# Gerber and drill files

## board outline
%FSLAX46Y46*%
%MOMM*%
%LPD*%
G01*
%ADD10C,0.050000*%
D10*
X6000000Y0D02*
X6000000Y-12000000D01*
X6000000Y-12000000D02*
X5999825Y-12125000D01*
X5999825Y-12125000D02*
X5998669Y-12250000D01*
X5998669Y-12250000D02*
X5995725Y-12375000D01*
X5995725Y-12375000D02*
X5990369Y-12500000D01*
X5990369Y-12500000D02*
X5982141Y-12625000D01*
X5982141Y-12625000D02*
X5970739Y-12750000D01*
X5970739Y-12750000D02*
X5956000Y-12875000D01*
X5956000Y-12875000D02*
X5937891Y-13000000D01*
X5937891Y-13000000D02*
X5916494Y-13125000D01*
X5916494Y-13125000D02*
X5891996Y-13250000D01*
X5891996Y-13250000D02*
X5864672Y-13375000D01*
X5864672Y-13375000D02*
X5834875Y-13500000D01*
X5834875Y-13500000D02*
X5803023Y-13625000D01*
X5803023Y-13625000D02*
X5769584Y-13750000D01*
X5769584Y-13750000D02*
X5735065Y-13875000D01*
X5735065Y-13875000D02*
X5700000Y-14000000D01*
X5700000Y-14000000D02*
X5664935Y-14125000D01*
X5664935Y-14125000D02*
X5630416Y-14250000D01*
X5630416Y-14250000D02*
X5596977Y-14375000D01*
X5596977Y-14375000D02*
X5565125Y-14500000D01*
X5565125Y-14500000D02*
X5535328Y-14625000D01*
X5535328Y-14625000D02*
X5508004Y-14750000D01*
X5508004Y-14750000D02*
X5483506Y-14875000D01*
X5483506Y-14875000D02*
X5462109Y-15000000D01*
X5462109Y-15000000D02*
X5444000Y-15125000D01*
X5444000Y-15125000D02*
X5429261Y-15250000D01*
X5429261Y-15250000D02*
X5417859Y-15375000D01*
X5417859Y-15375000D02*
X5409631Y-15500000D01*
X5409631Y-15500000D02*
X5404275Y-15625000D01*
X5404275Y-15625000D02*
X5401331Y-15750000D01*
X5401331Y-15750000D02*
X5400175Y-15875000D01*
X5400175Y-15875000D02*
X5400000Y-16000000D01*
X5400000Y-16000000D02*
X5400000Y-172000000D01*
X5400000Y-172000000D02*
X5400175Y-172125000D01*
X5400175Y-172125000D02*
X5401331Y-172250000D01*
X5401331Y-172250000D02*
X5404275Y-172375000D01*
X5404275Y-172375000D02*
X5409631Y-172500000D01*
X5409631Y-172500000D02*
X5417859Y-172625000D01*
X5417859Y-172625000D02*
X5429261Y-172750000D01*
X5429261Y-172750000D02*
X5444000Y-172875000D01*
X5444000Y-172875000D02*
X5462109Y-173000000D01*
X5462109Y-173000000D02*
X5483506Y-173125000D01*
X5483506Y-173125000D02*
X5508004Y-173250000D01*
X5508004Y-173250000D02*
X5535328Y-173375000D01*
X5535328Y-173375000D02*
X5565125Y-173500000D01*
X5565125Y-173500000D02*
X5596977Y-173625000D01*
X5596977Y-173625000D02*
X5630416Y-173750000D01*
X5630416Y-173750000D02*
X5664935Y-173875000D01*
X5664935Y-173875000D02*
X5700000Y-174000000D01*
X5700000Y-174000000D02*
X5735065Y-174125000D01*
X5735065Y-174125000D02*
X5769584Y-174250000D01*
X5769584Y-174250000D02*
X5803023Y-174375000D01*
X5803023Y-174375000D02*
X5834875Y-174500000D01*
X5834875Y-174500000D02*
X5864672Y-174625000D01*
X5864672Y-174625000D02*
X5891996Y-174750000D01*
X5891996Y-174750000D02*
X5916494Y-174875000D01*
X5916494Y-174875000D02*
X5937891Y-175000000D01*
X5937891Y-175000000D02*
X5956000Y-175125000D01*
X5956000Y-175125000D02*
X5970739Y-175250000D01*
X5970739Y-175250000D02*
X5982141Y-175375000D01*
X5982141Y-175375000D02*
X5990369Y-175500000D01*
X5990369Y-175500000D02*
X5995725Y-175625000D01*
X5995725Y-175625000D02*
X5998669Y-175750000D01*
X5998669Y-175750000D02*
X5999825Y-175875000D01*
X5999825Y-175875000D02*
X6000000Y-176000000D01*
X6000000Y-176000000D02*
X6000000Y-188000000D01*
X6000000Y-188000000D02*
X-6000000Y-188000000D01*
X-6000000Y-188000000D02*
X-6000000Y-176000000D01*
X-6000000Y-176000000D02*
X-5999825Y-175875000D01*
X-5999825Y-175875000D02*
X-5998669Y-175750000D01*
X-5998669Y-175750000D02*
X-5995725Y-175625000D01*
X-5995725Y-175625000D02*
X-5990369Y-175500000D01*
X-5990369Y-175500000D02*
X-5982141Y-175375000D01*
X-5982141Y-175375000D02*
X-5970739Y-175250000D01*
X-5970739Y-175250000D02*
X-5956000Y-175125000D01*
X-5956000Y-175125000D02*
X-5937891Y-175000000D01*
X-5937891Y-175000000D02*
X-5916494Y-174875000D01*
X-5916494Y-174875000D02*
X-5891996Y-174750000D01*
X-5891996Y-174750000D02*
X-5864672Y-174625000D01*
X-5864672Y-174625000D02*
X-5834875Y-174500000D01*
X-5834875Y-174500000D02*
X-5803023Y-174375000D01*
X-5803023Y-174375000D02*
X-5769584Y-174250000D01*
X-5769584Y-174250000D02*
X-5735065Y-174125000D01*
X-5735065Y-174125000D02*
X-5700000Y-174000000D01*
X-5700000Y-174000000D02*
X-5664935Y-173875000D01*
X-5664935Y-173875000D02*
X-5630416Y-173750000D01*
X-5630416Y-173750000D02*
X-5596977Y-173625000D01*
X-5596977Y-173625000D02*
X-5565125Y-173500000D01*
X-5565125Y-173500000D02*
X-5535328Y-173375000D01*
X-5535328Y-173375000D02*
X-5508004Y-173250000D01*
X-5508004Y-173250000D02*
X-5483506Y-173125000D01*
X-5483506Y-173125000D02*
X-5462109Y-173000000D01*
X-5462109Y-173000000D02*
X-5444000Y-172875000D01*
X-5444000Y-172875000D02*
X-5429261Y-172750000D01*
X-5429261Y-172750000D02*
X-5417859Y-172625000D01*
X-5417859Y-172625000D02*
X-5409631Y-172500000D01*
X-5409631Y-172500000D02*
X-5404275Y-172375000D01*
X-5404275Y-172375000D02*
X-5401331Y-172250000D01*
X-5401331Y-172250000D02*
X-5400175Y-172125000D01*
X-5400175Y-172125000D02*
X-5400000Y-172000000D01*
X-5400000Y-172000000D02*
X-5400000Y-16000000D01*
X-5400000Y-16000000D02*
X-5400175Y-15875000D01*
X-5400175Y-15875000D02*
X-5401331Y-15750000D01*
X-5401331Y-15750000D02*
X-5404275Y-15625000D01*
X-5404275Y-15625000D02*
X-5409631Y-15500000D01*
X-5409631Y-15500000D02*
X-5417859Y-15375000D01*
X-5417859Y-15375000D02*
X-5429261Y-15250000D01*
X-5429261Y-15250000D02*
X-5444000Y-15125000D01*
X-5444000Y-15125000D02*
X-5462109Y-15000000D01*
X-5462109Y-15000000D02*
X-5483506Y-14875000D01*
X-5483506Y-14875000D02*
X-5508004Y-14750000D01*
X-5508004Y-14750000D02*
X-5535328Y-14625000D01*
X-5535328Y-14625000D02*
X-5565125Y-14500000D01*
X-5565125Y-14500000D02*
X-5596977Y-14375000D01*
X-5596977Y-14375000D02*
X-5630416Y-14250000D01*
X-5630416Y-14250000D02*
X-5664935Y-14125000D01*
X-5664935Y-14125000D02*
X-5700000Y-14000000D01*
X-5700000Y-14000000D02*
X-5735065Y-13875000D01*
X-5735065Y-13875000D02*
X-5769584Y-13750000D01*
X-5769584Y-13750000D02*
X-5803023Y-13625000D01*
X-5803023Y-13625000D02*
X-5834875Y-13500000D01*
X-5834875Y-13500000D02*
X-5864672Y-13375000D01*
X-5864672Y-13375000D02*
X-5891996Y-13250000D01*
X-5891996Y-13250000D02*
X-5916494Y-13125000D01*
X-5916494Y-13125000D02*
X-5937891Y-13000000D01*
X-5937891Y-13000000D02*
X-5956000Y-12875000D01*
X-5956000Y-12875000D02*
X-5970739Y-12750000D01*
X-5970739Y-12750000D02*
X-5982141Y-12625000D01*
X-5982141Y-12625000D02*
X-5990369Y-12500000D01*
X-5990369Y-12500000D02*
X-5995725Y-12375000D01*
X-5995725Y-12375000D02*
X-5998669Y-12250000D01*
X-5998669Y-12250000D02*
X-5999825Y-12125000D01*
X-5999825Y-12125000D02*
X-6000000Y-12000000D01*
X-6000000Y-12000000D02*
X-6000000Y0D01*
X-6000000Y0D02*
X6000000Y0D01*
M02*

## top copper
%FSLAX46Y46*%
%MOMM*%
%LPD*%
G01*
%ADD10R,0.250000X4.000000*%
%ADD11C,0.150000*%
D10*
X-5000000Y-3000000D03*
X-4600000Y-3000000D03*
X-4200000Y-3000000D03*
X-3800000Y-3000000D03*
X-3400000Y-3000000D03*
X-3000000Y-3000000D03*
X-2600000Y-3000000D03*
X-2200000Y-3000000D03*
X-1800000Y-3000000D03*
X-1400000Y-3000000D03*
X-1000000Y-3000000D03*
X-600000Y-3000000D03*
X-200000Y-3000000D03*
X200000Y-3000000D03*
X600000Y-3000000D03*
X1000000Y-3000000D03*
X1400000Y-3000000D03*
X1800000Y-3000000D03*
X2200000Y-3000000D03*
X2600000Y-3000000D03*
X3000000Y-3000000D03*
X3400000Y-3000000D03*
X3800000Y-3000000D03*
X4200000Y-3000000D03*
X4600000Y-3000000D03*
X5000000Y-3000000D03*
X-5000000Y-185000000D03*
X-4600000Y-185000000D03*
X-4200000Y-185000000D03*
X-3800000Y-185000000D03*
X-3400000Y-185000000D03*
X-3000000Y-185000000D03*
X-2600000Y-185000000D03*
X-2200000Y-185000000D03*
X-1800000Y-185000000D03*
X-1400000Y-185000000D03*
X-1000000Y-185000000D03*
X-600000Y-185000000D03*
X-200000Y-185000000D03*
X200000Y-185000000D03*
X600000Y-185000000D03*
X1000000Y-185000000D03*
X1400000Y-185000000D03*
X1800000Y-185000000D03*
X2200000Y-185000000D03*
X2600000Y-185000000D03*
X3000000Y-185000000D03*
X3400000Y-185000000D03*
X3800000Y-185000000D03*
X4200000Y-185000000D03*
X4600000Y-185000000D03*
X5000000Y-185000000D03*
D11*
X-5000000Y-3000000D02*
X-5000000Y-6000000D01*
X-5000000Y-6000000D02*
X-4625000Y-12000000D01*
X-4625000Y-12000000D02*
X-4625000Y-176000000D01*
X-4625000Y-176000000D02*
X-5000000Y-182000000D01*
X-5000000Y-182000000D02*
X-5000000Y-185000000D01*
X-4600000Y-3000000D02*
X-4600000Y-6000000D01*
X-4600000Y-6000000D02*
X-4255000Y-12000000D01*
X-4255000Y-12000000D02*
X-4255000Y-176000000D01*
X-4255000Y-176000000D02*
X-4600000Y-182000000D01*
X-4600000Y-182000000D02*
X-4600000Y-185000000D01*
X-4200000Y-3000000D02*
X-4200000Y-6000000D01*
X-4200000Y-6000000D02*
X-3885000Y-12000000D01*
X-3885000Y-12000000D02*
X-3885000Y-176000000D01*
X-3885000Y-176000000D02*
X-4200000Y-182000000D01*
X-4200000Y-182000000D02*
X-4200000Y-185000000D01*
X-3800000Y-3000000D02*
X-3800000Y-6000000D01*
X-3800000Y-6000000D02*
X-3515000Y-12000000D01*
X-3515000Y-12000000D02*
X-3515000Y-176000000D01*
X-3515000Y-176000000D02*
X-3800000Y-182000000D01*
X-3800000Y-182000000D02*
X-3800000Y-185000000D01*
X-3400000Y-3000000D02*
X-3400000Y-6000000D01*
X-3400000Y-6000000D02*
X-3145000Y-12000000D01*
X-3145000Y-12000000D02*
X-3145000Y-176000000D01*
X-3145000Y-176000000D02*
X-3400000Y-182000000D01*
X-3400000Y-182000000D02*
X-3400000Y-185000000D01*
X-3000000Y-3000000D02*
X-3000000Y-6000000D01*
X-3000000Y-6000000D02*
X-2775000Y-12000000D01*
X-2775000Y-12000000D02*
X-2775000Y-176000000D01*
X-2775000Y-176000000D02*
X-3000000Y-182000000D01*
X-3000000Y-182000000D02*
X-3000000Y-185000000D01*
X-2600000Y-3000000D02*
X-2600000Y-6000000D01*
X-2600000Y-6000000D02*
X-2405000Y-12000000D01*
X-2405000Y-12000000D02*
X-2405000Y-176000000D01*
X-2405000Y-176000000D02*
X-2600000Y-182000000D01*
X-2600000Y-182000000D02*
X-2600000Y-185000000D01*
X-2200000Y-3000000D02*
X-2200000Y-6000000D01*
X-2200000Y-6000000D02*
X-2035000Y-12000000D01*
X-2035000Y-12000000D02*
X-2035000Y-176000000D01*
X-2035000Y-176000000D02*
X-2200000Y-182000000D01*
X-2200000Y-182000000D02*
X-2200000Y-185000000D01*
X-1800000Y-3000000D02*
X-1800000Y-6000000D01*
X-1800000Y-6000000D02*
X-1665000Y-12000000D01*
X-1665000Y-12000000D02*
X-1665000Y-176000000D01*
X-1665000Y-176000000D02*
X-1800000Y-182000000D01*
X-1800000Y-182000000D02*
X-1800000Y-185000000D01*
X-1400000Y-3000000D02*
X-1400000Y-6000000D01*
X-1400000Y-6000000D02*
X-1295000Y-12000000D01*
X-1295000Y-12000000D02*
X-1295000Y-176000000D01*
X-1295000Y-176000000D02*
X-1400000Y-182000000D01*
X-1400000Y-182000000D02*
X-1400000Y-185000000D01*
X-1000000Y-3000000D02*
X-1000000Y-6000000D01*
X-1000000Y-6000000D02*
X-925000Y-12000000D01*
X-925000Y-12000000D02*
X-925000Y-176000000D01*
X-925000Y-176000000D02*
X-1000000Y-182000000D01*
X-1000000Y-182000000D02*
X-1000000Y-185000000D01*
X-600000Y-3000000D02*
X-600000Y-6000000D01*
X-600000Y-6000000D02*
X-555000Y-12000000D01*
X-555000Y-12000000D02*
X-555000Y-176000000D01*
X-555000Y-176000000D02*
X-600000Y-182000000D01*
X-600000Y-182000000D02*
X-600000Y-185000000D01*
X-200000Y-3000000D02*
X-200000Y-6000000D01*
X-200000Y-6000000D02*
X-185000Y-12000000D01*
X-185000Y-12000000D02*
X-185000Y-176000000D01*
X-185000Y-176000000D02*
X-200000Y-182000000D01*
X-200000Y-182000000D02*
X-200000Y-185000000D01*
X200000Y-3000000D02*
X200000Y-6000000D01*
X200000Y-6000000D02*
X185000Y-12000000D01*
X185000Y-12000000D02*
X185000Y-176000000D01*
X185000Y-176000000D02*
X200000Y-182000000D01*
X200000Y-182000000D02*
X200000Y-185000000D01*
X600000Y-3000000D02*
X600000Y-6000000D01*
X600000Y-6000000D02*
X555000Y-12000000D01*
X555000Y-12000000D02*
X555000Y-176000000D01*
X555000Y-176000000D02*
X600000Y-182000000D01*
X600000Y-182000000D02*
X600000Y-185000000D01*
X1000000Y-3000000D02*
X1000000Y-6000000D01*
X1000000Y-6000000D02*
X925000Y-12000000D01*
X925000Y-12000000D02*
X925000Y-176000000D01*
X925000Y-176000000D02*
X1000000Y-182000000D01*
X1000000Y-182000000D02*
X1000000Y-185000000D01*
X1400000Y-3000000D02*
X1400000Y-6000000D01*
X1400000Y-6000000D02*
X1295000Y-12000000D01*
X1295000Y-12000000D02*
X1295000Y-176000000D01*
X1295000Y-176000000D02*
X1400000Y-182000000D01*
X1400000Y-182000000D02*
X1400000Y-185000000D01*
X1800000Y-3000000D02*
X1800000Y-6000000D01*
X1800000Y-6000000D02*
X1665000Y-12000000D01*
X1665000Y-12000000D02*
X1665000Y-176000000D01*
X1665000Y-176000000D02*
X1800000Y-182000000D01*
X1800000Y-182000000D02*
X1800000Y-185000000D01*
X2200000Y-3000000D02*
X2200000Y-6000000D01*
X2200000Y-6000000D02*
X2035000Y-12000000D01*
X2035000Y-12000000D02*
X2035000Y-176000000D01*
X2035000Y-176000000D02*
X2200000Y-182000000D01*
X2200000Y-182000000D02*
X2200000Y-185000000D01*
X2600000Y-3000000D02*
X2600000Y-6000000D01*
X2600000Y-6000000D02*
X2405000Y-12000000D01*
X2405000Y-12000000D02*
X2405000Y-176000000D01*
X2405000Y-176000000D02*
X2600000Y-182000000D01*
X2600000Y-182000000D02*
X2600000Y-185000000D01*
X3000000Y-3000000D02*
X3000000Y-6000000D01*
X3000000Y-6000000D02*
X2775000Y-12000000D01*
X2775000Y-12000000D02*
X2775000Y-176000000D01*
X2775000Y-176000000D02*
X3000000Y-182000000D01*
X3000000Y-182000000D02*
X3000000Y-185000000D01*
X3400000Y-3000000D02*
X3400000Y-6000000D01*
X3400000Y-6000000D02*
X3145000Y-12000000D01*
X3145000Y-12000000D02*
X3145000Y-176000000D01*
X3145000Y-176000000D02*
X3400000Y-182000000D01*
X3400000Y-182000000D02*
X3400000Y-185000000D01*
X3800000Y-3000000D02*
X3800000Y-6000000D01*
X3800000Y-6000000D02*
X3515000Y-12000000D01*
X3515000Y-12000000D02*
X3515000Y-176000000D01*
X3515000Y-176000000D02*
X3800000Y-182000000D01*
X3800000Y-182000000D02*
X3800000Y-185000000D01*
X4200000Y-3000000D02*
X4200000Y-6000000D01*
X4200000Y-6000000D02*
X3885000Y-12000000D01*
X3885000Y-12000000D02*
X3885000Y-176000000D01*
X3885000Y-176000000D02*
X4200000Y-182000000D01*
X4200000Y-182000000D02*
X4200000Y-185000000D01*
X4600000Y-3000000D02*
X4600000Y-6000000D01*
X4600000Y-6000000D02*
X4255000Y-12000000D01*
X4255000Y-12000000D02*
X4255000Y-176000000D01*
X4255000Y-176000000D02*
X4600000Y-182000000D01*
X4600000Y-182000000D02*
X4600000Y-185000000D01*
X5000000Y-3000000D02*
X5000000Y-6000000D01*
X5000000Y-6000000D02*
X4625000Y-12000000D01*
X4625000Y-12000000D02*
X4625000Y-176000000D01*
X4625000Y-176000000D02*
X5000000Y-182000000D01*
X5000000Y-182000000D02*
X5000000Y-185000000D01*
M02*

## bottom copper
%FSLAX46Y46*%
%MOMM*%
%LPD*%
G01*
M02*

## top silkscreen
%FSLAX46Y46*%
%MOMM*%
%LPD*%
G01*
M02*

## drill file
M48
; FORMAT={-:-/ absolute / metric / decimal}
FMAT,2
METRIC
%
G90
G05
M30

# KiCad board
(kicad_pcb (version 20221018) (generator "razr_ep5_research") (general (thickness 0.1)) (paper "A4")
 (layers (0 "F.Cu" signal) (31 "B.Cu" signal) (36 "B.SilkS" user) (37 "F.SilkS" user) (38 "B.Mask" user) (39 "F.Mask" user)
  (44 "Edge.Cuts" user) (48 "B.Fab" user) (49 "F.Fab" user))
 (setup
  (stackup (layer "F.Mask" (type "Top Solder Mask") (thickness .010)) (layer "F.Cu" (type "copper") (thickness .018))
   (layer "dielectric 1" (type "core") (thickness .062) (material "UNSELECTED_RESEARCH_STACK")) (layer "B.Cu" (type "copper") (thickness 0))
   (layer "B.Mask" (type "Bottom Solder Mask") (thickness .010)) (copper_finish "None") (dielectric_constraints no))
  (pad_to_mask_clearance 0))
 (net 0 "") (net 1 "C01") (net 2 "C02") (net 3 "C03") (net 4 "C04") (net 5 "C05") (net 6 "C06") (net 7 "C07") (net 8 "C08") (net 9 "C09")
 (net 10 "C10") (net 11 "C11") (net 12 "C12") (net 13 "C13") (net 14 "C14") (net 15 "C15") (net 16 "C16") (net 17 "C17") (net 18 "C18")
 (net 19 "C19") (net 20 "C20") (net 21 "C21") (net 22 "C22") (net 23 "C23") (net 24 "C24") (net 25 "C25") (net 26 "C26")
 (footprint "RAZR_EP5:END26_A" (layer "F.Cu") (at 0 0)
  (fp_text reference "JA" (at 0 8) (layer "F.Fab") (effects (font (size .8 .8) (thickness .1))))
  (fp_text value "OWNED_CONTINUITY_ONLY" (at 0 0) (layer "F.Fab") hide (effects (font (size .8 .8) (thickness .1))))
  (pad "1" smd rect (at -5.0 3.0) (size .25 4) (layers "F.Cu" "F.Mask") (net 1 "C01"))
  (pad "2" smd rect (at -4.6 3.0) (size .25 4) (layers "F.Cu" "F.Mask") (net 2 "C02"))
  (pad "3" smd rect (at -4.2 3.0) (size .25 4) (layers "F.Cu" "F.Mask") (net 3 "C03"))
  (pad "4" smd rect (at -3.8 3.0) (size .25 4) (layers "F.Cu" "F.Mask") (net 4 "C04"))
  (pad "5" smd rect (at -3.4 3.0) (size .25 4) (layers "F.Cu" "F.Mask") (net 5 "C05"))
  (pad "6" smd rect (at -3.0 3.0) (size .25 4) (layers "F.Cu" "F.Mask") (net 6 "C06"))
  (pad "7" smd rect (at -2.6 3.0) (size .25 4) (layers "F.Cu" "F.Mask") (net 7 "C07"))
  (pad "8" smd rect (at -2.2 3.0) (size .25 4) (layers "F.Cu" "F.Mask") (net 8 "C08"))
  (pad "9" smd rect (at -1.8 3.0) (size .25 4) (layers "F.Cu" "F.Mask") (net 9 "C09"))
  (pad "10" smd rect (at -1.4 3.0) (size .25 4) (layers "F.Cu" "F.Mask") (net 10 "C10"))
  (pad "11" smd rect (at -1.0 3.0) (size .25 4) (layers "F.Cu" "F.Mask") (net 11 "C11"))
  (pad "12" smd rect (at -0.6 3.0) (size .25 4) (layers "F.Cu" "F.Mask") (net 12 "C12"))
  (pad "13" smd rect (at -0.2 3.0) (size .25 4) (layers "F.Cu" "F.Mask") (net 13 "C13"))
  (pad "14" smd rect (at 0.2 3.0) (size .25 4) (layers "F.Cu" "F.Mask") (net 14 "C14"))
  (pad "15" smd rect (at 0.6 3.0) (size .25 4) (layers "F.Cu" "F.Mask") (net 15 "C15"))
  (pad "16" smd rect (at 1.0 3.0) (size .25 4) (layers "F.Cu" "F.Mask") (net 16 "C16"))
  (pad "17" smd rect (at 1.4 3.0) (size .25 4) (layers "F.Cu" "F.Mask") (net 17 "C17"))
  (pad "18" smd rect (at 1.8 3.0) (size .25 4) (layers "F.Cu" "F.Mask") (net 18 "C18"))
  (pad "19" smd rect (at 2.2 3.0) (size .25 4) (layers "F.Cu" "F.Mask") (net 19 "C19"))
  (pad "20" smd rect (at 2.6 3.0) (size .25 4) (layers "F.Cu" "F.Mask") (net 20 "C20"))
  (pad "21" smd rect (at 3.0 3.0) (size .25 4) (layers "F.Cu" "F.Mask") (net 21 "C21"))
  (pad "22" smd rect (at 3.4 3.0) (size .25 4) (layers "F.Cu" "F.Mask") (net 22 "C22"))
  (pad "23" smd rect (at 3.8 3.0) (size .25 4) (layers "F.Cu" "F.Mask") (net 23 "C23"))
  (pad "24" smd rect (at 4.2 3.0) (size .25 4) (layers "F.Cu" "F.Mask") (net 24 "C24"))
  (pad "25" smd rect (at 4.6 3.0) (size .25 4) (layers "F.Cu" "F.Mask") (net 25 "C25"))
  (pad "26" smd rect (at 5.0 3.0) (size .25 4) (layers "F.Cu" "F.Mask") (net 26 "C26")))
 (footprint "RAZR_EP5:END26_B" (layer "F.Cu") (at 0 0)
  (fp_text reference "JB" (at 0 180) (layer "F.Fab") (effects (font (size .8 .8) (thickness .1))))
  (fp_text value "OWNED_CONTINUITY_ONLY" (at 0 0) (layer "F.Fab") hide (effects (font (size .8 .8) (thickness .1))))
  (pad "1" smd rect (at -5.0 185.0) (size .25 4) (layers "F.Cu" "F.Mask") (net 1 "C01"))
  (pad "2" smd rect (at -4.6 185.0) (size .25 4) (layers "F.Cu" "F.Mask") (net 2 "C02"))
  (pad "3" smd rect (at -4.2 185.0) (size .25 4) (layers "F.Cu" "F.Mask") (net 3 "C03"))
  (pad "4" smd rect (at -3.8 185.0) (size .25 4) (layers "F.Cu" "F.Mask") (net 4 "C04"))
  (pad "5" smd rect (at -3.4 185.0) (size .25 4) (layers "F.Cu" "F.Mask") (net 5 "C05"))
  (pad "6" smd rect (at -3.0 185.0) (size .25 4) (layers "F.Cu" "F.Mask") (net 6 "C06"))
  (pad "7" smd rect (at -2.6 185.0) (size .25 4) (layers "F.Cu" "F.Mask") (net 7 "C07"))
  (pad "8" smd rect (at -2.2 185.0) (size .25 4) (layers "F.Cu" "F.Mask") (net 8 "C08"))
  (pad "9" smd rect (at -1.8 185.0) (size .25 4) (layers "F.Cu" "F.Mask") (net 9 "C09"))
  (pad "10" smd rect (at -1.4 185.0) (size .25 4) (layers "F.Cu" "F.Mask") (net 10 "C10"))
  (pad "11" smd rect (at -1.0 185.0) (size .25 4) (layers "F.Cu" "F.Mask") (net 11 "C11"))
  (pad "12" smd rect (at -0.6 185.0) (size .25 4) (layers "F.Cu" "F.Mask") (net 12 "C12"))
  (pad "13" smd rect (at -0.2 185.0) (size .25 4) (layers "F.Cu" "F.Mask") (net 13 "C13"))
  (pad "14" smd rect (at 0.2 185.0) (size .25 4) (layers "F.Cu" "F.Mask") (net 14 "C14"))
  (pad "15" smd rect (at 0.6 185.0) (size .25 4) (layers "F.Cu" "F.Mask") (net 15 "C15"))
  (pad "16" smd rect (at 1.0 185.0) (size .25 4) (layers "F.Cu" "F.Mask") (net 16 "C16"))
  (pad "17" smd rect (at 1.4 185.0) (size .25 4) (layers "F.Cu" "F.Mask") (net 17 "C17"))
  (pad "18" smd rect (at 1.8 185.0) (size .25 4) (layers "F.Cu" "F.Mask") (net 18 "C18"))
  (pad "19" smd rect (at 2.2 185.0) (size .25 4) (layers "F.Cu" "F.Mask") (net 19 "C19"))
  (pad "20" smd rect (at 2.6 185.0) (size .25 4) (layers "F.Cu" "F.Mask") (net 20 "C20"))
  (pad "21" smd rect (at 3.0 185.0) (size .25 4) (layers "F.Cu" "F.Mask") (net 21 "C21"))
  (pad "22" smd rect (at 3.4 185.0) (size .25 4) (layers "F.Cu" "F.Mask") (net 22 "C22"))
  (pad "23" smd rect (at 3.8 185.0) (size .25 4) (layers "F.Cu" "F.Mask") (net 23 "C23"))
  (pad "24" smd rect (at 4.2 185.0) (size .25 4) (layers "F.Cu" "F.Mask") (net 24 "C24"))
  (pad "25" smd rect (at 4.6 185.0) (size .25 4) (layers "F.Cu" "F.Mask") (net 25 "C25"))
  (pad "26" smd rect (at 5.0 185.0) (size .25 4) (layers "F.Cu" "F.Mask") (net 26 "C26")))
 (segment (start -5.0 3.0) (end -5.0 6.0) (width .15) (layer "F.Cu") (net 1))
 (segment (start -5.0 6.0) (end -4.625 12) (width .15) (layer "F.Cu") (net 1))
 (segment (start -4.625 12) (end -4.625 176) (width .15) (layer "F.Cu") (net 1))
 (segment (start -4.625 176) (end -5.0 182.0) (width .15) (layer "F.Cu") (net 1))
 (segment (start -5.0 182.0) (end -5.0 185.0) (width .15) (layer "F.Cu") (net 1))
 (segment (start -4.6 3.0) (end -4.6 6.0) (width .15) (layer "F.Cu") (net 2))
 (segment (start -4.6 6.0) (end -4.255 12) (width .15) (layer "F.Cu") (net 2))
 (segment (start -4.255 12) (end -4.255 176) (width .15) (layer "F.Cu") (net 2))
 (segment (start -4.255 176) (end -4.6 182.0) (width .15) (layer "F.Cu") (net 2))
 (segment (start -4.6 182.0) (end -4.6 185.0) (width .15) (layer "F.Cu") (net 2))
 (segment (start -4.2 3.0) (end -4.2 6.0) (width .15) (layer "F.Cu") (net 3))
 (segment (start -4.2 6.0) (end -3.885 12) (width .15) (layer "F.Cu") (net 3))
 (segment (start -3.885 12) (end -3.885 176) (width .15) (layer "F.Cu") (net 3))
 (segment (start -3.885 176) (end -4.2 182.0) (width .15) (layer "F.Cu") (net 3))
 (segment (start -4.2 182.0) (end -4.2 185.0) (width .15) (layer "F.Cu") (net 3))
 (segment (start -3.8 3.0) (end -3.8 6.0) (width .15) (layer "F.Cu") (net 4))
 (segment (start -3.8 6.0) (end -3.515 12) (width .15) (layer "F.Cu") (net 4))
 (segment (start -3.515 12) (end -3.515 176) (width .15) (layer "F.Cu") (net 4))
 (segment (start -3.515 176) (end -3.8 182.0) (width .15) (layer "F.Cu") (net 4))
 (segment (start -3.8 182.0) (end -3.8 185.0) (width .15) (layer "F.Cu") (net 4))
 (segment (start -3.4 3.0) (end -3.4 6.0) (width .15) (layer "F.Cu") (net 5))
 (segment (start -3.4 6.0) (end -3.145 12) (width .15) (layer "F.Cu") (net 5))
 (segment (start -3.145 12) (end -3.145 176) (width .15) (layer "F.Cu") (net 5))
 (segment (start -3.145 176) (end -3.4 182.0) (width .15) (layer "F.Cu") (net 5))
 (segment (start -3.4 182.0) (end -3.4 185.0) (width .15) (layer "F.Cu") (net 5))
 (segment (start -3.0 3.0) (end -3.0 6.0) (width .15) (layer "F.Cu") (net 6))
 (segment (start -3.0 6.0) (end -2.775 12) (width .15) (layer "F.Cu") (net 6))
 (segment (start -2.775 12) (end -2.775 176) (width .15) (layer "F.Cu") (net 6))
 (segment (start -2.775 176) (end -3.0 182.0) (width .15) (layer "F.Cu") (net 6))
 (segment (start -3.0 182.0) (end -3.0 185.0) (width .15) (layer "F.Cu") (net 6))
 (segment (start -2.6 3.0) (end -2.6 6.0) (width .15) (layer "F.Cu") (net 7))
 (segment (start -2.6 6.0) (end -2.405 12) (width .15) (layer "F.Cu") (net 7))
 (segment (start -2.405 12) (end -2.405 176) (width .15) (layer "F.Cu") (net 7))
 (segment (start -2.405 176) (end -2.6 182.0) (width .15) (layer "F.Cu") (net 7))
 (segment (start -2.6 182.0) (end -2.6 185.0) (width .15) (layer "F.Cu") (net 7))
 (segment (start -2.2 3.0) (end -2.2 6.0) (width .15) (layer "F.Cu") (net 8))
 (segment (start -2.2 6.0) (end -2.035 12) (width .15) (layer "F.Cu") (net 8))
 (segment (start -2.035 12) (end -2.035 176) (width .15) (layer "F.Cu") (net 8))
 (segment (start -2.035 176) (end -2.2 182.0) (width .15) (layer "F.Cu") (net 8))
 (segment (start -2.2 182.0) (end -2.2 185.0) (width .15) (layer "F.Cu") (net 8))
 (segment (start -1.8 3.0) (end -1.8 6.0) (width .15) (layer "F.Cu") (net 9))
 (segment (start -1.8 6.0) (end -1.665 12) (width .15) (layer "F.Cu") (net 9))
 (segment (start -1.665 12) (end -1.665 176) (width .15) (layer "F.Cu") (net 9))
 (segment (start -1.665 176) (end -1.8 182.0) (width .15) (layer "F.Cu") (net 9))
 (segment (start -1.8 182.0) (end -1.8 185.0) (width .15) (layer "F.Cu") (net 9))
 (segment (start -1.4 3.0) (end -1.4 6.0) (width .15) (layer "F.Cu") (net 10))
 (segment (start -1.4 6.0) (end -1.295 12) (width .15) (layer "F.Cu") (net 10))
 (segment (start -1.295 12) (end -1.295 176) (width .15) (layer "F.Cu") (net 10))
 (segment (start -1.295 176) (end -1.4 182.0) (width .15) (layer "F.Cu") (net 10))
 (segment (start -1.4 182.0) (end -1.4 185.0) (width .15) (layer "F.Cu") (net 10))
 (segment (start -1.0 3.0) (end -1.0 6.0) (width .15) (layer "F.Cu") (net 11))
 (segment (start -1.0 6.0) (end -0.925 12) (width .15) (layer "F.Cu") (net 11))
 (segment (start -0.925 12) (end -0.925 176) (width .15) (layer "F.Cu") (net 11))
 (segment (start -0.925 176) (end -1.0 182.0) (width .15) (layer "F.Cu") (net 11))
 (segment (start -1.0 182.0) (end -1.0 185.0) (width .15) (layer "F.Cu") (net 11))
 (segment (start -0.6 3.0) (end -0.6 6.0) (width .15) (layer "F.Cu") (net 12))
 (segment (start -0.6 6.0) (end -0.555 12) (width .15) (layer "F.Cu") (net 12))
 (segment (start -0.555 12) (end -0.555 176) (width .15) (layer "F.Cu") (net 12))
 (segment (start -0.555 176) (end -0.6 182.0) (width .15) (layer "F.Cu") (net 12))
 (segment (start -0.6 182.0) (end -0.6 185.0) (width .15) (layer "F.Cu") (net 12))
 (segment (start -0.2 3.0) (end -0.2 6.0) (width .15) (layer "F.Cu") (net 13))
 (segment (start -0.2 6.0) (end -0.185 12) (width .15) (layer "F.Cu") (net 13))
 (segment (start -0.185 12) (end -0.185 176) (width .15) (layer "F.Cu") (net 13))
 (segment (start -0.185 176) (end -0.2 182.0) (width .15) (layer "F.Cu") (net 13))
 (segment (start -0.2 182.0) (end -0.2 185.0) (width .15) (layer "F.Cu") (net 13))
 (segment (start 0.2 3.0) (end 0.2 6.0) (width .15) (layer "F.Cu") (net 14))
 (segment (start 0.2 6.0) (end 0.185 12) (width .15) (layer "F.Cu") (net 14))
 (segment (start 0.185 12) (end 0.185 176) (width .15) (layer "F.Cu") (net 14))
 (segment (start 0.185 176) (end 0.2 182.0) (width .15) (layer "F.Cu") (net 14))
 (segment (start 0.2 182.0) (end 0.2 185.0) (width .15) (layer "F.Cu") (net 14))
 (segment (start 0.6 3.0) (end 0.6 6.0) (width .15) (layer "F.Cu") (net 15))
 (segment (start 0.6 6.0) (end 0.555 12) (width .15) (layer "F.Cu") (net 15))
 (segment (start 0.555 12) (end 0.555 176) (width .15) (layer "F.Cu") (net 15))
 (segment (start 0.555 176) (end 0.6 182.0) (width .15) (layer "F.Cu") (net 15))
 (segment (start 0.6 182.0) (end 0.6 185.0) (width .15) (layer "F.Cu") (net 15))
 (segment (start 1.0 3.0) (end 1.0 6.0) (width .15) (layer "F.Cu") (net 16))
 (segment (start 1.0 6.0) (end 0.925 12) (width .15) (layer "F.Cu") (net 16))
 (segment (start 0.925 12) (end 0.925 176) (width .15) (layer "F.Cu") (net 16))
 (segment (start 0.925 176) (end 1.0 182.0) (width .15) (layer "F.Cu") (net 16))
 (segment (start 1.0 182.0) (end 1.0 185.0) (width .15) (layer "F.Cu") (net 16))
 (segment (start 1.4 3.0) (end 1.4 6.0) (width .15) (layer "F.Cu") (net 17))
 (segment (start 1.4 6.0) (end 1.295 12) (width .15) (layer "F.Cu") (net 17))
 (segment (start 1.295 12) (end 1.295 176) (width .15) (layer "F.Cu") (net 17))
 (segment (start 1.295 176) (end 1.4 182.0) (width .15) (layer "F.Cu") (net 17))
 (segment (start 1.4 182.0) (end 1.4 185.0) (width .15) (layer "F.Cu") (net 17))
 (segment (start 1.8 3.0) (end 1.8 6.0) (width .15) (layer "F.Cu") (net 18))
 (segment (start 1.8 6.0) (end 1.665 12) (width .15) (layer "F.Cu") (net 18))
 (segment (start 1.665 12) (end 1.665 176) (width .15) (layer "F.Cu") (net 18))
 (segment (start 1.665 176) (end 1.8 182.0) (width .15) (layer "F.Cu") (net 18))
 (segment (start 1.8 182.0) (end 1.8 185.0) (width .15) (layer "F.Cu") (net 18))
 (segment (start 2.2 3.0) (end 2.2 6.0) (width .15) (layer "F.Cu") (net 19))
 (segment (start 2.2 6.0) (end 2.035 12) (width .15) (layer "F.Cu") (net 19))
 (segment (start 2.035 12) (end 2.035 176) (width .15) (layer "F.Cu") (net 19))
 (segment (start 2.035 176) (end 2.2 182.0) (width .15) (layer "F.Cu") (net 19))
 (segment (start 2.2 182.0) (end 2.2 185.0) (width .15) (layer "F.Cu") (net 19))
 (segment (start 2.6 3.0) (end 2.6 6.0) (width .15) (layer "F.Cu") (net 20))
 (segment (start 2.6 6.0) (end 2.405 12) (width .15) (layer "F.Cu") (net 20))
 (segment (start 2.405 12) (end 2.405 176) (width .15) (layer "F.Cu") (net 20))
 (segment (start 2.405 176) (end 2.6 182.0) (width .15) (layer "F.Cu") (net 20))
 (segment (start 2.6 182.0) (end 2.6 185.0) (width .15) (layer "F.Cu") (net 20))
 (segment (start 3.0 3.0) (end 3.0 6.0) (width .15) (layer "F.Cu") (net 21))
 (segment (start 3.0 6.0) (end 2.775 12) (width .15) (layer "F.Cu") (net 21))
 (segment (start 2.775 12) (end 2.775 176) (width .15) (layer "F.Cu") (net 21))
 (segment (start 2.775 176) (end 3.0 182.0) (width .15) (layer "F.Cu") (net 21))
 (segment (start 3.0 182.0) (end 3.0 185.0) (width .15) (layer "F.Cu") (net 21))
 (segment (start 3.4 3.0) (end 3.4 6.0) (width .15) (layer "F.Cu") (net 22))
 (segment (start 3.4 6.0) (end 3.145 12) (width .15) (layer "F.Cu") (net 22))
 (segment (start 3.145 12) (end 3.145 176) (width .15) (layer "F.Cu") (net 22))
 (segment (start 3.145 176) (end 3.4 182.0) (width .15) (layer "F.Cu") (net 22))
 (segment (start 3.4 182.0) (end 3.4 185.0) (width .15) (layer "F.Cu") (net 22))
 (segment (start 3.8 3.0) (end 3.8 6.0) (width .15) (layer "F.Cu") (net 23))
 (segment (start 3.8 6.0) (end 3.515 12) (width .15) (layer "F.Cu") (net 23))
 (segment (start 3.515 12) (end 3.515 176) (width .15) (layer "F.Cu") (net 23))
 (segment (start 3.515 176) (end 3.8 182.0) (width .15) (layer "F.Cu") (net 23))
 (segment (start 3.8 182.0) (end 3.8 185.0) (width .15) (layer "F.Cu") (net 23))
 (segment (start 4.2 3.0) (end 4.2 6.0) (width .15) (layer "F.Cu") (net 24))
 (segment (start 4.2 6.0) (end 3.885 12) (width .15) (layer "F.Cu") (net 24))
 (segment (start 3.885 12) (end 3.885 176) (width .15) (layer "F.Cu") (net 24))
 (segment (start 3.885 176) (end 4.2 182.0) (width .15) (layer "F.Cu") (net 24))
 (segment (start 4.2 182.0) (end 4.2 185.0) (width .15) (layer "F.Cu") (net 24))
 (segment (start 4.6 3.0) (end 4.6 6.0) (width .15) (layer "F.Cu") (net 25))
 (segment (start 4.6 6.0) (end 4.255 12) (width .15) (layer "F.Cu") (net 25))
 (segment (start 4.255 12) (end 4.255 176) (width .15) (layer "F.Cu") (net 25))
 (segment (start 4.255 176) (end 4.6 182.0) (width .15) (layer "F.Cu") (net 25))
 (segment (start 4.6 182.0) (end 4.6 185.0) (width .15) (layer "F.Cu") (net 25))
 (segment (start 5.0 3.0) (end 5.0 6.0) (width .15) (layer "F.Cu") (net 26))
 (segment (start 5.0 6.0) (end 4.625 12) (width .15) (layer "F.Cu") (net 26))
 (segment (start 4.625 12) (end 4.625 176) (width .15) (layer "F.Cu") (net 26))
 (segment (start 4.625 176) (end 5.0 182.0) (width .15) (layer "F.Cu") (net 26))
 (segment (start 5.0 182.0) (end 5.0 185.0) (width .15) (layer "F.Cu") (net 26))
 (gr_line (start 6.0 0.0) (end 6.0 12) (layer "Edge.Cuts") (width .05))
 (gr_line (start 6.0 12) (end 5.99982537 12.125) (layer "Edge.Cuts") (width .05))
 (gr_line (start 5.99982537 12.125) (end 5.998669052 12.25) (layer "Edge.Cuts") (width .05))
 (gr_line (start 5.998669052 12.25) (end 5.99572531 12.375) (layer "Edge.Cuts") (width .05))
 (gr_line (start 5.99572531 12.375) (end 5.990368652 12.5) (layer "Edge.Cuts") (width .05))
 (gr_line (start 5.990368652 12.5) (end 5.982140958 12.625) (layer "Edge.Cuts") (width .05))
 (gr_line (start 5.982140958 12.625) (end 5.970738602 12.75) (layer "Edge.Cuts") (width .05))
 (gr_line (start 5.970738602 12.75) (end 5.955999577 12.875) (layer "Edge.Cuts") (width .05))
 (gr_line (start 5.955999577 12.875) (end 5.937890625 13.0) (layer "Edge.Cuts") (width .05))
 (gr_line (start 5.937890625 13.0) (end 5.916494358 13.125) (layer "Edge.Cuts") (width .05))
 (gr_line (start 5.916494358 13.125) (end 5.891996384 13.25) (layer "Edge.Cuts") (width .05))
 (gr_line (start 5.891996384 13.25) (end 5.864672434 13.375) (layer "Edge.Cuts") (width .05))
 (gr_line (start 5.864672434 13.375) (end 5.834875488 13.5) (layer "Edge.Cuts") (width .05))
 (gr_line (start 5.834875488 13.5) (end 5.803022897 13.625) (layer "Edge.Cuts") (width .05))
 (gr_line (start 5.803022897 13.625) (end 5.769583511 13.75) (layer "Edge.Cuts") (width .05))
 (gr_line (start 5.769583511 13.75) (end 5.735064805 13.875) (layer "Edge.Cuts") (width .05))
 (gr_line (start 5.735064805 13.875) (end 5.7 14.0) (layer "Edge.Cuts") (width .05))
 (gr_line (start 5.7 14.0) (end 5.664935195 14.125) (layer "Edge.Cuts") (width .05))
 (gr_line (start 5.664935195 14.125) (end 5.630416489 14.25) (layer "Edge.Cuts") (width .05))
 (gr_line (start 5.630416489 14.25) (end 5.596977103 14.375) (layer "Edge.Cuts") (width .05))
 (gr_line (start 5.596977103 14.375) (end 5.565124512 14.5) (layer "Edge.Cuts") (width .05))
 (gr_line (start 5.565124512 14.5) (end 5.535327566 14.625) (layer "Edge.Cuts") (width .05))
 (gr_line (start 5.535327566 14.625) (end 5.508003616 14.75) (layer "Edge.Cuts") (width .05))
 (gr_line (start 5.508003616 14.75) (end 5.483505642 14.875) (layer "Edge.Cuts") (width .05))
 (gr_line (start 5.483505642 14.875) (end 5.462109375 15.0) (layer "Edge.Cuts") (width .05))
 (gr_line (start 5.462109375 15.0) (end 5.444000423 15.125) (layer "Edge.Cuts") (width .05))
 (gr_line (start 5.444000423 15.125) (end 5.429261398 15.25) (layer "Edge.Cuts") (width .05))
 (gr_line (start 5.429261398 15.25) (end 5.417859042 15.375) (layer "Edge.Cuts") (width .05))
 (gr_line (start 5.417859042 15.375) (end 5.409631348 15.5) (layer "Edge.Cuts") (width .05))
 (gr_line (start 5.409631348 15.5) (end 5.40427469 15.625) (layer "Edge.Cuts") (width .05))
 (gr_line (start 5.40427469 15.625) (end 5.401330948 15.75) (layer "Edge.Cuts") (width .05))
 (gr_line (start 5.401330948 15.75) (end 5.40017463 15.875) (layer "Edge.Cuts") (width .05))
 (gr_line (start 5.40017463 15.875) (end 5.4 16.0) (layer "Edge.Cuts") (width .05))
 (gr_line (start 5.4 16.0) (end 5.4 172.0) (layer "Edge.Cuts") (width .05))
 (gr_line (start 5.4 172.0) (end 5.40017463 172.125) (layer "Edge.Cuts") (width .05))
 (gr_line (start 5.40017463 172.125) (end 5.401330948 172.25) (layer "Edge.Cuts") (width .05))
 (gr_line (start 5.401330948 172.25) (end 5.40427469 172.375) (layer "Edge.Cuts") (width .05))
 (gr_line (start 5.40427469 172.375) (end 5.409631348 172.5) (layer "Edge.Cuts") (width .05))
 (gr_line (start 5.409631348 172.5) (end 5.417859042 172.625) (layer "Edge.Cuts") (width .05))
 (gr_line (start 5.417859042 172.625) (end 5.429261398 172.75) (layer "Edge.Cuts") (width .05))
 (gr_line (start 5.429261398 172.75) (end 5.444000423 172.875) (layer "Edge.Cuts") (width .05))
 (gr_line (start 5.444000423 172.875) (end 5.462109375 173.0) (layer "Edge.Cuts") (width .05))
 (gr_line (start 5.462109375 173.0) (end 5.483505642 173.125) (layer "Edge.Cuts") (width .05))
 (gr_line (start 5.483505642 173.125) (end 5.508003616 173.25) (layer "Edge.Cuts") (width .05))
 (gr_line (start 5.508003616 173.25) (end 5.535327566 173.375) (layer "Edge.Cuts") (width .05))
 (gr_line (start 5.535327566 173.375) (end 5.565124512 173.5) (layer "Edge.Cuts") (width .05))
 (gr_line (start 5.565124512 173.5) (end 5.596977103 173.625) (layer "Edge.Cuts") (width .05))
 (gr_line (start 5.596977103 173.625) (end 5.630416489 173.75) (layer "Edge.Cuts") (width .05))
 (gr_line (start 5.630416489 173.75) (end 5.664935195 173.875) (layer "Edge.Cuts") (width .05))
 (gr_line (start 5.664935195 173.875) (end 5.7 174.0) (layer "Edge.Cuts") (width .05))
 (gr_line (start 5.7 174.0) (end 5.735064805 174.125) (layer "Edge.Cuts") (width .05))
 (gr_line (start 5.735064805 174.125) (end 5.769583511 174.25) (layer "Edge.Cuts") (width .05))
 (gr_line (start 5.769583511 174.25) (end 5.803022897 174.375) (layer "Edge.Cuts") (width .05))
 (gr_line (start 5.803022897 174.375) (end 5.834875488 174.5) (layer "Edge.Cuts") (width .05))
 (gr_line (start 5.834875488 174.5) (end 5.864672434 174.625) (layer "Edge.Cuts") (width .05))
 (gr_line (start 5.864672434 174.625) (end 5.891996384 174.75) (layer "Edge.Cuts") (width .05))
 (gr_line (start 5.891996384 174.75) (end 5.916494358 174.875) (layer "Edge.Cuts") (width .05))
 (gr_line (start 5.916494358 174.875) (end 5.937890625 175.0) (layer "Edge.Cuts") (width .05))
 (gr_line (start 5.937890625 175.0) (end 5.955999577 175.125) (layer "Edge.Cuts") (width .05))
 (gr_line (start 5.955999577 175.125) (end 5.970738602 175.25) (layer "Edge.Cuts") (width .05))
 (gr_line (start 5.970738602 175.25) (end 5.982140958 175.375) (layer "Edge.Cuts") (width .05))
 (gr_line (start 5.982140958 175.375) (end 5.990368652 175.5) (layer "Edge.Cuts") (width .05))
 (gr_line (start 5.990368652 175.5) (end 5.99572531 175.625) (layer "Edge.Cuts") (width .05))
 (gr_line (start 5.99572531 175.625) (end 5.998669052 175.75) (layer "Edge.Cuts") (width .05))
 (gr_line (start 5.998669052 175.75) (end 5.99982537 175.875) (layer "Edge.Cuts") (width .05))
 (gr_line (start 5.99982537 175.875) (end 6.0 176) (layer "Edge.Cuts") (width .05))
 (gr_line (start 6.0 176) (end 6.0 188) (layer "Edge.Cuts") (width .05))
 (gr_line (start 6.0 188) (end -6.0 188) (layer "Edge.Cuts") (width .05))
 (gr_line (start -6.0 188) (end -6.0 176) (layer "Edge.Cuts") (width .05))
 (gr_line (start -6.0 176) (end -5.99982537 175.875) (layer "Edge.Cuts") (width .05))
 (gr_line (start -5.99982537 175.875) (end -5.998669052 175.75) (layer "Edge.Cuts") (width .05))
 (gr_line (start -5.998669052 175.75) (end -5.99572531 175.625) (layer "Edge.Cuts") (width .05))
 (gr_line (start -5.99572531 175.625) (end -5.990368652 175.5) (layer "Edge.Cuts") (width .05))
 (gr_line (start -5.990368652 175.5) (end -5.982140958 175.375) (layer "Edge.Cuts") (width .05))
 (gr_line (start -5.982140958 175.375) (end -5.970738602 175.25) (layer "Edge.Cuts") (width .05))
 (gr_line (start -5.970738602 175.25) (end -5.955999577 175.125) (layer "Edge.Cuts") (width .05))
 (gr_line (start -5.955999577 175.125) (end -5.937890625 175.0) (layer "Edge.Cuts") (width .05))
 (gr_line (start -5.937890625 175.0) (end -5.916494358 174.875) (layer "Edge.Cuts") (width .05))
 (gr_line (start -5.916494358 174.875) (end -5.891996384 174.75) (layer "Edge.Cuts") (width .05))
 (gr_line (start -5.891996384 174.75) (end -5.864672434 174.625) (layer "Edge.Cuts") (width .05))
 (gr_line (start -5.864672434 174.625) (end -5.834875488 174.5) (layer "Edge.Cuts") (width .05))
 (gr_line (start -5.834875488 174.5) (end -5.803022897 174.375) (layer "Edge.Cuts") (width .05))
 (gr_line (start -5.803022897 174.375) (end -5.769583511 174.25) (layer "Edge.Cuts") (width .05))
 (gr_line (start -5.769583511 174.25) (end -5.735064805 174.125) (layer "Edge.Cuts") (width .05))
 (gr_line (start -5.735064805 174.125) (end -5.7 174.0) (layer "Edge.Cuts") (width .05))
 (gr_line (start -5.7 174.0) (end -5.664935195 173.875) (layer "Edge.Cuts") (width .05))
 (gr_line (start -5.664935195 173.875) (end -5.630416489 173.75) (layer "Edge.Cuts") (width .05))
 (gr_line (start -5.630416489 173.75) (end -5.596977103 173.625) (layer "Edge.Cuts") (width .05))
 (gr_line (start -5.596977103 173.625) (end -5.565124512 173.5) (layer "Edge.Cuts") (width .05))
 (gr_line (start -5.565124512 173.5) (end -5.535327566 173.375) (layer "Edge.Cuts") (width .05))
 (gr_line (start -5.535327566 173.375) (end -5.508003616 173.25) (layer "Edge.Cuts") (width .05))
 (gr_line (start -5.508003616 173.25) (end -5.483505642 173.125) (layer "Edge.Cuts") (width .05))
 (gr_line (start -5.483505642 173.125) (end -5.462109375 173.0) (layer "Edge.Cuts") (width .05))
 (gr_line (start -5.462109375 173.0) (end -5.444000423 172.875) (layer "Edge.Cuts") (width .05))
 (gr_line (start -5.444000423 172.875) (end -5.429261398 172.75) (layer "Edge.Cuts") (width .05))
 (gr_line (start -5.429261398 172.75) (end -5.417859042 172.625) (layer "Edge.Cuts") (width .05))
 (gr_line (start -5.417859042 172.625) (end -5.409631348 172.5) (layer "Edge.Cuts") (width .05))
 (gr_line (start -5.409631348 172.5) (end -5.40427469 172.375) (layer "Edge.Cuts") (width .05))
 (gr_line (start -5.40427469 172.375) (end -5.401330948 172.25) (layer "Edge.Cuts") (width .05))
 (gr_line (start -5.401330948 172.25) (end -5.40017463 172.125) (layer "Edge.Cuts") (width .05))
 (gr_line (start -5.40017463 172.125) (end -5.4 172.0) (layer "Edge.Cuts") (width .05))
 (gr_line (start -5.4 172.0) (end -5.4 16.0) (layer "Edge.Cuts") (width .05))
 (gr_line (start -5.4 16.0) (end -5.40017463 15.875) (layer "Edge.Cuts") (width .05))
 (gr_line (start -5.40017463 15.875) (end -5.401330948 15.75) (layer "Edge.Cuts") (width .05))
 (gr_line (start -5.401330948 15.75) (end -5.40427469 15.625) (layer "Edge.Cuts") (width .05))
 (gr_line (start -5.40427469 15.625) (end -5.409631348 15.5) (layer "Edge.Cuts") (width .05))
 (gr_line (start -5.409631348 15.5) (end -5.417859042 15.375) (layer "Edge.Cuts") (width .05))
 (gr_line (start -5.417859042 15.375) (end -5.429261398 15.25) (layer "Edge.Cuts") (width .05))
 (gr_line (start -5.429261398 15.25) (end -5.444000423 15.125) (layer "Edge.Cuts") (width .05))
 (gr_line (start -5.444000423 15.125) (end -5.462109375 15.0) (layer "Edge.Cuts") (width .05))
 (gr_line (start -5.462109375 15.0) (end -5.483505642 14.875) (layer "Edge.Cuts") (width .05))
 (gr_line (start -5.483505642 14.875) (end -5.508003616 14.75) (layer "Edge.Cuts") (width .05))
 (gr_line (start -5.508003616 14.75) (end -5.535327566 14.625) (layer "Edge.Cuts") (width .05))
 (gr_line (start -5.535327566 14.625) (end -5.565124512 14.5) (layer "Edge.Cuts") (width .05))
 (gr_line (start -5.565124512 14.5) (end -5.596977103 14.375) (layer "Edge.Cuts") (width .05))
 (gr_line (start -5.596977103 14.375) (end -5.630416489 14.25) (layer "Edge.Cuts") (width .05))
 (gr_line (start -5.630416489 14.25) (end -5.664935195 14.125) (layer "Edge.Cuts") (width .05))
 (gr_line (start -5.664935195 14.125) (end -5.7 14.0) (layer "Edge.Cuts") (width .05))
 (gr_line (start -5.7 14.0) (end -5.735064805 13.875) (layer "Edge.Cuts") (width .05))
 (gr_line (start -5.735064805 13.875) (end -5.769583511 13.75) (layer "Edge.Cuts") (width .05))
 (gr_line (start -5.769583511 13.75) (end -5.803022897 13.625) (layer "Edge.Cuts") (width .05))
 (gr_line (start -5.803022897 13.625) (end -5.834875488 13.5) (layer "Edge.Cuts") (width .05))
 (gr_line (start -5.834875488 13.5) (end -5.864672434 13.375) (layer "Edge.Cuts") (width .05))
 (gr_line (start -5.864672434 13.375) (end -5.891996384 13.25) (layer "Edge.Cuts") (width .05))
 (gr_line (start -5.891996384 13.25) (end -5.916494358 13.125) (layer "Edge.Cuts") (width .05))
 (gr_line (start -5.916494358 13.125) (end -5.937890625 13.0) (layer "Edge.Cuts") (width .05))
 (gr_line (start -5.937890625 13.0) (end -5.955999577 12.875) (layer "Edge.Cuts") (width .05))
 (gr_line (start -5.955999577 12.875) (end -5.970738602 12.75) (layer "Edge.Cuts") (width .05))
 (gr_line (start -5.970738602 12.75) (end -5.982140958 12.625) (layer "Edge.Cuts") (width .05))
 (gr_line (start -5.982140958 12.625) (end -5.990368652 12.5) (layer "Edge.Cuts") (width .05))
 (gr_line (start -5.990368652 12.5) (end -5.99572531 12.375) (layer "Edge.Cuts") (width .05))
 (gr_line (start -5.99572531 12.375) (end -5.998669052 12.25) (layer "Edge.Cuts") (width .05))
 (gr_line (start -5.998669052 12.25) (end -5.99982537 12.125) (layer "Edge.Cuts") (width .05))
 (gr_line (start -5.99982537 12.125) (end -6.0 12) (layer "Edge.Cuts") (width .05))
 (gr_line (start -6.0 12) (end -6.0 0.0) (layer "Edge.Cuts") (width .05))
 (gr_line (start -6.0 0.0) (end 6.0 0.0) (layer "Edge.Cuts") (width .05)))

